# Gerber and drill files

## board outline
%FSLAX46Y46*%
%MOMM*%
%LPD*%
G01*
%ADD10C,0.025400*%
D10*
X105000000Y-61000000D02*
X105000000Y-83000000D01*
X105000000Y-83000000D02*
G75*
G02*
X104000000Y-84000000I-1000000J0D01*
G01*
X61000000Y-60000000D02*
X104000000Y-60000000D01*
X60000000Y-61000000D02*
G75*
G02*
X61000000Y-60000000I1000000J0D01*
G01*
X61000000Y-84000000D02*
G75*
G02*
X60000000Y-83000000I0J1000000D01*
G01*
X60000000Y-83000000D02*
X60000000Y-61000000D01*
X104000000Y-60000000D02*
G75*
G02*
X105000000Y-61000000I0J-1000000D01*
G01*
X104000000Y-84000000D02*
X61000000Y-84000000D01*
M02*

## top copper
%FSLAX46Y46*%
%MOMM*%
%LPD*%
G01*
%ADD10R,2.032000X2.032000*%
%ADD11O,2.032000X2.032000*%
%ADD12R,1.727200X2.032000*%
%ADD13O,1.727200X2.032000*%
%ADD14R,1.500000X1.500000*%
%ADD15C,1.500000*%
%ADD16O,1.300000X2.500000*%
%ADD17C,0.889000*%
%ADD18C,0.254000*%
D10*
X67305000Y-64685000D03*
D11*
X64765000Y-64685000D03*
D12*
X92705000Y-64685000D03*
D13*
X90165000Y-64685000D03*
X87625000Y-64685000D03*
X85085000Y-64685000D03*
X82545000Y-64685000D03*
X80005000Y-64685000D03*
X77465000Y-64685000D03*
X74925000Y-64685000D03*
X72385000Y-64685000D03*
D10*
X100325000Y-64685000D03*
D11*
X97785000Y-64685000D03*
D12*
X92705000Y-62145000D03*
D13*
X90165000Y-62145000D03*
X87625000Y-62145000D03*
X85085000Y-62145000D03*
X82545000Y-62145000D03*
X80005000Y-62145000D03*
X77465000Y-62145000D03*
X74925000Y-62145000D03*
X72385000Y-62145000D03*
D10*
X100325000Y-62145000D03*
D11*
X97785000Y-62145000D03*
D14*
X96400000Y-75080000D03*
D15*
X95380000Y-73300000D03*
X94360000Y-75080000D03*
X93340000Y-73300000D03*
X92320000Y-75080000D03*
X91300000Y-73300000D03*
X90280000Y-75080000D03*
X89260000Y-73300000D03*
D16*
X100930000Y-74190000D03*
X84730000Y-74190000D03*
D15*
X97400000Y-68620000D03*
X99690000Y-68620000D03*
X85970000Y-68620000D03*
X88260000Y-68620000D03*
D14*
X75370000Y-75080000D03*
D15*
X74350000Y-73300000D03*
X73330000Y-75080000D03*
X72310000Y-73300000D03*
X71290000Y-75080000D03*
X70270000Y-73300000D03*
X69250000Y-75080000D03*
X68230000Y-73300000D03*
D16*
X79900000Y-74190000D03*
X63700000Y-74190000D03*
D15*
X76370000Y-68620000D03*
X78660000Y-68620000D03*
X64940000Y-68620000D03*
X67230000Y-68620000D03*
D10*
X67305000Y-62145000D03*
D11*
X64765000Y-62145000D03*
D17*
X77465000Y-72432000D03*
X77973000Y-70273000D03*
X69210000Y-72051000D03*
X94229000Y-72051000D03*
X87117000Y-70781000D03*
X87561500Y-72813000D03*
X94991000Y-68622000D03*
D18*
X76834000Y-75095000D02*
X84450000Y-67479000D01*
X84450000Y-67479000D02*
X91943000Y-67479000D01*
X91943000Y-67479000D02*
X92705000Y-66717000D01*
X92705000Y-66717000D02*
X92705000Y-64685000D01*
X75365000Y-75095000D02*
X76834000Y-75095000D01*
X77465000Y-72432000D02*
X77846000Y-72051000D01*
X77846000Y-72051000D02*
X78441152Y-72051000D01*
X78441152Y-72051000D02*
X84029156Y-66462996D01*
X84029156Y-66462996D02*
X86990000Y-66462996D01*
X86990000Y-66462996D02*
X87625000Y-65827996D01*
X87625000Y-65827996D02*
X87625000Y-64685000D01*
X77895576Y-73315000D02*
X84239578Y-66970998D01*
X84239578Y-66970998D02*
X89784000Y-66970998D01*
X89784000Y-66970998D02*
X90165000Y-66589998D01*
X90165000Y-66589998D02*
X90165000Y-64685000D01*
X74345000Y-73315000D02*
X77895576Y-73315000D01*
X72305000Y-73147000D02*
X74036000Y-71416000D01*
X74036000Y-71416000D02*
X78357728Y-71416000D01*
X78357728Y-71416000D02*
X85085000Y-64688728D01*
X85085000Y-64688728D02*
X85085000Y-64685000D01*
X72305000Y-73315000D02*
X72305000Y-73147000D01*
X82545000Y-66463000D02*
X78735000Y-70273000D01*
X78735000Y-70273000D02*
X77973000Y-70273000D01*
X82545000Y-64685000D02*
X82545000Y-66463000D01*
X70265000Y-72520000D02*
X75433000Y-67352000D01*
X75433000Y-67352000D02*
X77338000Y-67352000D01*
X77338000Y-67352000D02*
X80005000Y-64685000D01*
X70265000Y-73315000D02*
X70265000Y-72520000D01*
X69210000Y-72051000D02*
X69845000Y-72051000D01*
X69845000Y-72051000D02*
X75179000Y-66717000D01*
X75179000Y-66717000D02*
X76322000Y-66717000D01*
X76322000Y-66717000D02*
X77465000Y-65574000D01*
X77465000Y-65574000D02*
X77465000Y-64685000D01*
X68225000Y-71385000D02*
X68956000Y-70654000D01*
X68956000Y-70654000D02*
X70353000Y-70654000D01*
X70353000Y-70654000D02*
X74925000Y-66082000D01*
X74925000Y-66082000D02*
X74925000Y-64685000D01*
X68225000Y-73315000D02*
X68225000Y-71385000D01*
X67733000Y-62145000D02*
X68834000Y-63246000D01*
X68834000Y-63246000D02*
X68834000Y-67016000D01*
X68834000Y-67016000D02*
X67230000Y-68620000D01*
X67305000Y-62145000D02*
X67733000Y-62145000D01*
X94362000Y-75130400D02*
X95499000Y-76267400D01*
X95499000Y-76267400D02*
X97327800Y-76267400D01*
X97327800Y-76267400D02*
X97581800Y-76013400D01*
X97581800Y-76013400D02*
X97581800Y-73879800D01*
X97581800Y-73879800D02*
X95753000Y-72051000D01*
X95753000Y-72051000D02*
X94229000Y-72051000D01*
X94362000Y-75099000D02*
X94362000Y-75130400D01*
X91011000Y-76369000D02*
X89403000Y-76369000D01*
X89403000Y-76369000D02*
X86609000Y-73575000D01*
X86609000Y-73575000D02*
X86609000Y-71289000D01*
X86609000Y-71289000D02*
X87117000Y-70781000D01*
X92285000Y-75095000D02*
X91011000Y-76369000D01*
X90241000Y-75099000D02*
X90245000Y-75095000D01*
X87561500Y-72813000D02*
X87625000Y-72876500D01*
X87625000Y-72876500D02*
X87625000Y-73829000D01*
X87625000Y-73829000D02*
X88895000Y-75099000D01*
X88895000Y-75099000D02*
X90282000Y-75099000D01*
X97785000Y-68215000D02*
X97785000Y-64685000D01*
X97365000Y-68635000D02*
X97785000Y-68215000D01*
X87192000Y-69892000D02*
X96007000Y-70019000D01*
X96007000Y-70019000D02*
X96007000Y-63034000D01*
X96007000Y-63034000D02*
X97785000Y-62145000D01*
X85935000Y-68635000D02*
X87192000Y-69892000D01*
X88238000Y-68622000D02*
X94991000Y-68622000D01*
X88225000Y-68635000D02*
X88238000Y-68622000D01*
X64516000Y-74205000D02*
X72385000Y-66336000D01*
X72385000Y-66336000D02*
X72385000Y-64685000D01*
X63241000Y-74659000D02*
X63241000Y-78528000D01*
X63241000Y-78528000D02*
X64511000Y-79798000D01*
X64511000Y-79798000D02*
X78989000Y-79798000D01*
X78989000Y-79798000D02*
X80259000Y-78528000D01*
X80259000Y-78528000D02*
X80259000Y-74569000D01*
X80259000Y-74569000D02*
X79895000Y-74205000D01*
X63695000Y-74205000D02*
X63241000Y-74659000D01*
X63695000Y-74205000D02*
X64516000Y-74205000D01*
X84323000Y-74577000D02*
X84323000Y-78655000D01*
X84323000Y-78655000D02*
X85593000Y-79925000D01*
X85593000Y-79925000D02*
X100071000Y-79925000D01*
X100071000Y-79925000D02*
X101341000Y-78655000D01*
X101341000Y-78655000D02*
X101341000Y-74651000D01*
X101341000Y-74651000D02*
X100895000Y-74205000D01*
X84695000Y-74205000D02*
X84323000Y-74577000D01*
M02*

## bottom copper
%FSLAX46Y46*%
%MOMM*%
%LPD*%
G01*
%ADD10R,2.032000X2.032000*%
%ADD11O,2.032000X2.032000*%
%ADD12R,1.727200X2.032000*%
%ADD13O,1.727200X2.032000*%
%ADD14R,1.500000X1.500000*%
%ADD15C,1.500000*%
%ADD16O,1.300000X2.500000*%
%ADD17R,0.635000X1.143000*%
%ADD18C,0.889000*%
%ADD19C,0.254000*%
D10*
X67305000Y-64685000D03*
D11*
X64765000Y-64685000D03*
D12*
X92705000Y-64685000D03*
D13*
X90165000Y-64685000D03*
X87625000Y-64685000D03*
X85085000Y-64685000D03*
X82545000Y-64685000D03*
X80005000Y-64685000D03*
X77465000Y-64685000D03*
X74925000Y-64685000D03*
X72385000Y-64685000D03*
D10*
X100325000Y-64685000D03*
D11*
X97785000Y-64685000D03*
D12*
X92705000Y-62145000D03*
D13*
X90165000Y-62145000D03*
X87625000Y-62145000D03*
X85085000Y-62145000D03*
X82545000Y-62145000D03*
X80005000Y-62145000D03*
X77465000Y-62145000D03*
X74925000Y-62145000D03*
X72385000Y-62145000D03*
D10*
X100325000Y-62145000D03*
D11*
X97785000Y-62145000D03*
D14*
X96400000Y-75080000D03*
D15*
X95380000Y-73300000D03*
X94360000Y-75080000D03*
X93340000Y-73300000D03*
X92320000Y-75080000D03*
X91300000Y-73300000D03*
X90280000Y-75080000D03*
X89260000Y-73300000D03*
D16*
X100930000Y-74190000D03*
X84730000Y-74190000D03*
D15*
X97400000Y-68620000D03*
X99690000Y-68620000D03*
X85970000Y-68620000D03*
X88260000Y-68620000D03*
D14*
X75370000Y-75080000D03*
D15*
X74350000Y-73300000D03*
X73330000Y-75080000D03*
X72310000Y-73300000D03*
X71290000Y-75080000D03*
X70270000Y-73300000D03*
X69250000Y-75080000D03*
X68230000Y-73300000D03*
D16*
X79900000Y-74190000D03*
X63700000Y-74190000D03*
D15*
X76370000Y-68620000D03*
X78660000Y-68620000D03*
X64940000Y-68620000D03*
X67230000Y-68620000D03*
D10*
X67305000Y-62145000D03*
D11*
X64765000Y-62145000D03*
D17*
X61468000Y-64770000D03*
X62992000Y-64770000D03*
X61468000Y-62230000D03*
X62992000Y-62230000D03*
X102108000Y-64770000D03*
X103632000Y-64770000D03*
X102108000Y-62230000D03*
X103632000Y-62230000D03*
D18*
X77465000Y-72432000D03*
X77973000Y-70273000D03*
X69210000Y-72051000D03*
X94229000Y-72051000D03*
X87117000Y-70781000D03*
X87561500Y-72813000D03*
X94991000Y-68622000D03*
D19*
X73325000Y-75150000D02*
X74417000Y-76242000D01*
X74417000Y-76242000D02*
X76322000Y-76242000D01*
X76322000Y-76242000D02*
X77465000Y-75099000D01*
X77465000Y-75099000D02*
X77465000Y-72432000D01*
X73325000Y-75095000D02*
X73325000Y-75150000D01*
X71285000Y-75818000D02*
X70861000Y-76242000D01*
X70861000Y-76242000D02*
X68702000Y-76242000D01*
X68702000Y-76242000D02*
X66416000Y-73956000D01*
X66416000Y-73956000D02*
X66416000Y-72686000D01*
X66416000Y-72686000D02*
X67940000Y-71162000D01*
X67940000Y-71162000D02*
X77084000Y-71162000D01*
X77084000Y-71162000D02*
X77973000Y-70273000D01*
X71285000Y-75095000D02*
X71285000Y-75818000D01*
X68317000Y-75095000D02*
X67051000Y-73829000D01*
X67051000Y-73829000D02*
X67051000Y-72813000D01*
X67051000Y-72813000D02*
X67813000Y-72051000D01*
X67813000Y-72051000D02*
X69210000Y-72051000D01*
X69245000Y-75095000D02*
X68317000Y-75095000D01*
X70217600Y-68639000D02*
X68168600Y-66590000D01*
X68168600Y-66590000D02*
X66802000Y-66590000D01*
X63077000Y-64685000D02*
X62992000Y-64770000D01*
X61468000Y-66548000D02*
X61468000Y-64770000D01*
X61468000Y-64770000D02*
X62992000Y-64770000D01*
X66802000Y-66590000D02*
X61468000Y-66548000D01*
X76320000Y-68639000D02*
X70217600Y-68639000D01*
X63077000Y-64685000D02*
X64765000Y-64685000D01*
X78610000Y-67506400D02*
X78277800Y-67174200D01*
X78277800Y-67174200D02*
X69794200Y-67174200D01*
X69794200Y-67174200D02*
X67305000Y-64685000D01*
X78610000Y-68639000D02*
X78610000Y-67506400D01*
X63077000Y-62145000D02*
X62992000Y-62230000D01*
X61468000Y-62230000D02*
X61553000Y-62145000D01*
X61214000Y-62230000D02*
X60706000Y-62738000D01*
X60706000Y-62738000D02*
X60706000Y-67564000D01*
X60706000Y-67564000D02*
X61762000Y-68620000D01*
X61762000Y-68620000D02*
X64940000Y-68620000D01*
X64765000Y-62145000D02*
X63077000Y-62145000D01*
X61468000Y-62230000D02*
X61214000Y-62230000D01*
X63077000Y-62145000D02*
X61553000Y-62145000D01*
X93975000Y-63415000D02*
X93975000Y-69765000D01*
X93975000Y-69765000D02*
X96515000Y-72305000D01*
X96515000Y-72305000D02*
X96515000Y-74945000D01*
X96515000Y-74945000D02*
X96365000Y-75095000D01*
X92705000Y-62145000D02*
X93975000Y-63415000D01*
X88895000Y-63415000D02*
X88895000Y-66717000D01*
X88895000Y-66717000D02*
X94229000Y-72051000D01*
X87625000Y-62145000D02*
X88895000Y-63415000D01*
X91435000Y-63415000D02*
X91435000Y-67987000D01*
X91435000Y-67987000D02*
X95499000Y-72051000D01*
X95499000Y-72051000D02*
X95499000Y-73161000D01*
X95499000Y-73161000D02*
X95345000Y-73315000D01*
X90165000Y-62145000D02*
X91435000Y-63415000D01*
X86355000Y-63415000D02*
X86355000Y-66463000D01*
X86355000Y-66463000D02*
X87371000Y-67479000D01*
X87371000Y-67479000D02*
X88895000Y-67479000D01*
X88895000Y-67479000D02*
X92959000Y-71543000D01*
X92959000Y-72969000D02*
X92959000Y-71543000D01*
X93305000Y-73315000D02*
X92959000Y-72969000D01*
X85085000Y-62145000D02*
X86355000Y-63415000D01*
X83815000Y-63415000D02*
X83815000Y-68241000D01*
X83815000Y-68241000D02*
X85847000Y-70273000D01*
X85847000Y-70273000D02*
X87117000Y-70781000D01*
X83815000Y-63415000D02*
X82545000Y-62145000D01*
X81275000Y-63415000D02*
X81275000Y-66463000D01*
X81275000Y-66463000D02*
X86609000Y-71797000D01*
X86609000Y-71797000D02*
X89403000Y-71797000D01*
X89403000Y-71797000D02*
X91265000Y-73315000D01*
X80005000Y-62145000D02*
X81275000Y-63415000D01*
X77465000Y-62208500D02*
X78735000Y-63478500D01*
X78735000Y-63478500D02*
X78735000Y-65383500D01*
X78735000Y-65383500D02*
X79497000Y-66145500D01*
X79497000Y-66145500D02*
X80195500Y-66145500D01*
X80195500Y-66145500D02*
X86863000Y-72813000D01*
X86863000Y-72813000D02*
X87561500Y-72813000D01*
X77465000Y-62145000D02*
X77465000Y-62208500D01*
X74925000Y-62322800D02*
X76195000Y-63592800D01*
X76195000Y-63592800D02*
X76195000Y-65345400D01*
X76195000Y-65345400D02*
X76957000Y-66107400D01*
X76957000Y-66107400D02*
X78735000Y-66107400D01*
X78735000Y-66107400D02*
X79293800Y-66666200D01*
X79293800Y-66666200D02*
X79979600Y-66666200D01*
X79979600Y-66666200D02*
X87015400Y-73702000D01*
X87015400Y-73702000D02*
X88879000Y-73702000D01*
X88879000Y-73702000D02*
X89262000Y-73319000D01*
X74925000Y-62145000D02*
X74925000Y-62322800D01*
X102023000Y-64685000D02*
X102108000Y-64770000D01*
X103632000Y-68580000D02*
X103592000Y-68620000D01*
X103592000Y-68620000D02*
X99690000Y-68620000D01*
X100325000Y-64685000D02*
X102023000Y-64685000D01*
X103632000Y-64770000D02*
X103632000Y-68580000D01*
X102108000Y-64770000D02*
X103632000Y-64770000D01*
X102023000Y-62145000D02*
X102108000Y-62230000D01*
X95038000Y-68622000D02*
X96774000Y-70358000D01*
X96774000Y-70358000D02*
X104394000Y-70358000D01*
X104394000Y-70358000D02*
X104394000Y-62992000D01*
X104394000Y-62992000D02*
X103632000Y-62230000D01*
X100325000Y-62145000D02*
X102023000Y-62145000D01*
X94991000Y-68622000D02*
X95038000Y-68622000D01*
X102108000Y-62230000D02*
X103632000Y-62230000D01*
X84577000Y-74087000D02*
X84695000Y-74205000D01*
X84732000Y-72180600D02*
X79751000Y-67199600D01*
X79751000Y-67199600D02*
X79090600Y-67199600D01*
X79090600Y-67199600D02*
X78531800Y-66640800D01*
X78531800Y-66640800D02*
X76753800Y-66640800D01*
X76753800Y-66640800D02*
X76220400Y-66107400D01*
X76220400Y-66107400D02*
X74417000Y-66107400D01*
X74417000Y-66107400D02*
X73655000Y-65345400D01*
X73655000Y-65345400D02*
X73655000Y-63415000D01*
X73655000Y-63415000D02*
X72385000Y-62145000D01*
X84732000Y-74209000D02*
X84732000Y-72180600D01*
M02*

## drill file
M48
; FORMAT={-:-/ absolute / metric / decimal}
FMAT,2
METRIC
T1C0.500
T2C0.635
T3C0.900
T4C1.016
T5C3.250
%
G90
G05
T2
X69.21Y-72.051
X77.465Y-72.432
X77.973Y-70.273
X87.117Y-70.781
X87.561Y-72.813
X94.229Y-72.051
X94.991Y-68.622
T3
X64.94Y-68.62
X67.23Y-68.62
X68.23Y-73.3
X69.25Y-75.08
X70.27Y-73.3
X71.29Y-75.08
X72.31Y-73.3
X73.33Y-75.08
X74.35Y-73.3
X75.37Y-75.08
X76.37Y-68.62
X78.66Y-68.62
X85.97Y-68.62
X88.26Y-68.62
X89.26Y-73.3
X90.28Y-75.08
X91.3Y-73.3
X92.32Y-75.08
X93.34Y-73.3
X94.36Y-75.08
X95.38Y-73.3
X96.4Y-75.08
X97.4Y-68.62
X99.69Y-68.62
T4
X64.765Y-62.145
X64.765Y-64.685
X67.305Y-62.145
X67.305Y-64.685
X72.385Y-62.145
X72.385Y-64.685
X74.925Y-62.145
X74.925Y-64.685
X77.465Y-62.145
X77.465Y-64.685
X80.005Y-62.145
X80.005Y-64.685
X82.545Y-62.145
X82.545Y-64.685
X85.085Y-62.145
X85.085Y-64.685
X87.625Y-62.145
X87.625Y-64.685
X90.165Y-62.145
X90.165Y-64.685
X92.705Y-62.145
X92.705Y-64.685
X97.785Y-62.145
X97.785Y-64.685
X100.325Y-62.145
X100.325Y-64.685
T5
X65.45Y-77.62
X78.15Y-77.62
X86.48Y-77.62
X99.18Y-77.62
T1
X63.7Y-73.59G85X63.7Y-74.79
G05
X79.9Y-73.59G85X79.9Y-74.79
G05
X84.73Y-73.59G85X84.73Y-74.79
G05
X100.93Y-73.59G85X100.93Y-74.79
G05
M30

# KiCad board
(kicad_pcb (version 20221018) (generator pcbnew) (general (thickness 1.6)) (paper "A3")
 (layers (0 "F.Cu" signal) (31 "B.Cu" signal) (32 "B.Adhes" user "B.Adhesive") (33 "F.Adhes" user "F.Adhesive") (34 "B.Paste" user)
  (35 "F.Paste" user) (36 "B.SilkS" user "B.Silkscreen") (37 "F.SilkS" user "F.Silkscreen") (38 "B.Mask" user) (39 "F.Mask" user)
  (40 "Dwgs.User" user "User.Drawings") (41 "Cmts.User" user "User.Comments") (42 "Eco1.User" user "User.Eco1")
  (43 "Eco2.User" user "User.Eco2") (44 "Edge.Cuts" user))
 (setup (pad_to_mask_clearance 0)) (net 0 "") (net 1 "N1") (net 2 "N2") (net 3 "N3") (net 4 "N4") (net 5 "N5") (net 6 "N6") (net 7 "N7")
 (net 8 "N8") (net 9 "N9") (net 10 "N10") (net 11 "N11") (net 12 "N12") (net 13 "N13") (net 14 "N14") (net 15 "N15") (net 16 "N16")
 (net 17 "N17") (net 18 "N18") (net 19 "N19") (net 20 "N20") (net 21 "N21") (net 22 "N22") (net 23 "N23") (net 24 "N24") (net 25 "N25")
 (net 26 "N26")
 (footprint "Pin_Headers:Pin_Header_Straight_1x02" (layer "F.Cu") (at 66.035 64.685 180)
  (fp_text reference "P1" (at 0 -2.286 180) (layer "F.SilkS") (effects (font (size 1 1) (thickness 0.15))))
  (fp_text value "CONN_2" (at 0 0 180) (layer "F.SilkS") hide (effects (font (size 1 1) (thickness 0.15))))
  (pad "1" thru_hole rect (at -1.27 0 180) (size 2.032 2.032) (drill 1.016) (layers "*.Cu" "*.Mask" "F.SilkS") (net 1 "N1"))
  (pad "2" thru_hole oval (at 1.27 0 180) (size 2.032 2.032) (drill 1.016) (layers "*.Cu" "*.Mask" "F.SilkS") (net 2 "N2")))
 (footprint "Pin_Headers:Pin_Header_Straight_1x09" (layer "F.Cu") (at 82.545 64.685 180)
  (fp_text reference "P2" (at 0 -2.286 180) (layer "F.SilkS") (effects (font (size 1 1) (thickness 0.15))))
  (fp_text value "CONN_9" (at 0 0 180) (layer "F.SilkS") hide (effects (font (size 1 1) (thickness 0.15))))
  (pad "1" thru_hole rect (at -10.16 0 180) (size 1.7272 2.032) (drill 1.016) (layers "*.Cu" "*.Mask" "F.SilkS") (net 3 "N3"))
  (pad "2" thru_hole oval (at -7.62 0 180) (size 1.7272 2.032) (drill 1.016) (layers "*.Cu" "*.Mask" "F.SilkS") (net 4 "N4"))
  (pad "3" thru_hole oval (at -5.08 0 180) (size 1.7272 2.032) (drill 1.016) (layers "*.Cu" "*.Mask" "F.SilkS") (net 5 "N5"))
  (pad "4" thru_hole oval (at -2.54 0 180) (size 1.7272 2.032) (drill 1.016) (layers "*.Cu" "*.Mask" "F.SilkS") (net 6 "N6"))
  (pad "5" thru_hole oval (at 0 0 180) (size 1.7272 2.032) (drill 1.016) (layers "*.Cu" "*.Mask" "F.SilkS") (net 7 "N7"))
  (pad "6" thru_hole oval (at 2.54 0 180) (size 1.7272 2.032) (drill 1.016) (layers "*.Cu" "*.Mask" "F.SilkS") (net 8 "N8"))
  (pad "7" thru_hole oval (at 5.08 0 180) (size 1.7272 2.032) (drill 1.016) (layers "*.Cu" "*.Mask" "F.SilkS") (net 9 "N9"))
  (pad "8" thru_hole oval (at 7.62 0 180) (size 1.7272 2.032) (drill 1.016) (layers "*.Cu" "*.Mask" "F.SilkS") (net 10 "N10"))
  (pad "9" thru_hole oval (at 10.16 0 180) (size 1.7272 2.032) (drill 1.016) (layers "*.Cu" "*.Mask" "F.SilkS") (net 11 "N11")))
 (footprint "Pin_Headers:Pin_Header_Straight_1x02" (layer "F.Cu") (at 99.055 64.685 180)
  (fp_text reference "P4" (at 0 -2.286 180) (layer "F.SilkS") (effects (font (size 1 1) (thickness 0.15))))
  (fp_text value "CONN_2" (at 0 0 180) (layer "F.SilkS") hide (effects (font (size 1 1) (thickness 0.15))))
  (pad "1" thru_hole rect (at -1.27 0 180) (size 2.032 2.032) (drill 1.016) (layers "*.Cu" "*.Mask" "F.SilkS") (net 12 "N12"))
  (pad "2" thru_hole oval (at 1.27 0 180) (size 2.032 2.032) (drill 1.016) (layers "*.Cu" "*.Mask" "F.SilkS") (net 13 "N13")))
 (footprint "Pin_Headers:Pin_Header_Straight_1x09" (layer "F.Cu") (at 82.545 62.145 180)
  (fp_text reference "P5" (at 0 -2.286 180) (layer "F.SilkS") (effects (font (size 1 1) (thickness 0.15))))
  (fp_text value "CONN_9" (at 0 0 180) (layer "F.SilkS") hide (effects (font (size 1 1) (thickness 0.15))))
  (pad "1" thru_hole rect (at -10.16 0 180) (size 1.7272 2.032) (drill 1.016) (layers "*.Cu" "*.Mask" "F.SilkS") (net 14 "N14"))
  (pad "2" thru_hole oval (at -7.62 0 180) (size 1.7272 2.032) (drill 1.016) (layers "*.Cu" "*.Mask" "F.SilkS") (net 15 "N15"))
  (pad "3" thru_hole oval (at -5.08 0 180) (size 1.7272 2.032) (drill 1.016) (layers "*.Cu" "*.Mask" "F.SilkS") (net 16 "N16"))
  (pad "4" thru_hole oval (at -2.54 0 180) (size 1.7272 2.032) (drill 1.016) (layers "*.Cu" "*.Mask" "F.SilkS") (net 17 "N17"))
  (pad "5" thru_hole oval (at 0 0 180) (size 1.7272 2.032) (drill 1.016) (layers "*.Cu" "*.Mask" "F.SilkS") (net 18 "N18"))
  (pad "6" thru_hole oval (at 2.54 0 180) (size 1.7272 2.032) (drill 1.016) (layers "*.Cu" "*.Mask" "F.SilkS") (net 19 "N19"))
  (pad "7" thru_hole oval (at 5.08 0 180) (size 1.7272 2.032) (drill 1.016) (layers "*.Cu" "*.Mask" "F.SilkS") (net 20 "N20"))
  (pad "8" thru_hole oval (at 7.62 0 180) (size 1.7272 2.032) (drill 1.016) (layers "*.Cu" "*.Mask" "F.SilkS") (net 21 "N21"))
  (pad "9" thru_hole oval (at 10.16 0 180) (size 1.7272 2.032) (drill 1.016) (layers "*.Cu" "*.Mask" "F.SilkS") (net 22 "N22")))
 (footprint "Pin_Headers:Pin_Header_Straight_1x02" (layer "F.Cu") (at 99.055 62.145 180)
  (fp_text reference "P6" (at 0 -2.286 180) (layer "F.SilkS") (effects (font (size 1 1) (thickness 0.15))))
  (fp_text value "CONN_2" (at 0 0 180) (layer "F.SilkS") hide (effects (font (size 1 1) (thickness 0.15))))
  (pad "1" thru_hole rect (at -1.27 0 180) (size 2.032 2.032) (drill 1.016) (layers "*.Cu" "*.Mask" "F.SilkS") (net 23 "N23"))
  (pad "2" thru_hole oval (at 1.27 0 180) (size 2.032 2.032) (drill 1.016) (layers "*.Cu" "*.Mask" "F.SilkS") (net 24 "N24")))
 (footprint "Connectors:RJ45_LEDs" (layer "F.Cu") (at 96.4 75.08 180)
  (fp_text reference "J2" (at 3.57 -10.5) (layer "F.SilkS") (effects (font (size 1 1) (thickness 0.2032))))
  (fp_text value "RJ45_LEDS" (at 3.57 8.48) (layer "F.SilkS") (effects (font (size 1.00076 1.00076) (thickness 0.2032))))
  (pad "" np_thru_hole circle (at -2.78 -2.54) (size 3.25 3.25) (drill 3.25) (layers "*.Cu" "*.Mask" "F.SilkS"))
  (pad "" np_thru_hole circle (at 9.92 -2.54) (size 3.25 3.25) (drill 3.25) (layers "*.Cu" "*.Mask" "F.SilkS"))
  (pad "1" thru_hole rect (at 0 0) (size 1.5 1.5) (drill 0.9) (layers "*.Cu" "*.Mask" "F.SilkS") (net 14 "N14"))
  (pad "2" thru_hole circle (at 1.02 1.78) (size 1.5 1.5) (drill 0.9) (layers "*.Cu" "*.Mask" "F.SilkS") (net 15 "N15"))
  (pad "3" thru_hole circle (at 2.04 0) (size 1.5 1.5) (drill 0.9) (layers "*.Cu" "*.Mask" "F.SilkS") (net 16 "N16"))
  (pad "4" thru_hole circle (at 3.06 1.78) (size 1.5 1.5) (drill 0.9) (layers "*.Cu" "*.Mask" "F.SilkS") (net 17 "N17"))
  (pad "5" thru_hole circle (at 4.08 0) (size 1.5 1.5) (drill 0.9) (layers "*.Cu" "*.Mask" "F.SilkS") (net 18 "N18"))
  (pad "6" thru_hole circle (at 5.1 1.78) (size 1.5 1.5) (drill 0.9) (layers "*.Cu" "*.Mask" "F.SilkS") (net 19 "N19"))
  (pad "7" thru_hole circle (at 6.12 0) (size 1.5 1.5) (drill 0.9) (layers "*.Cu" "*.Mask" "F.SilkS") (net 20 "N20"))
  (pad "8" thru_hole circle (at 7.14 1.78) (size 1.5 1.5) (drill 0.9) (layers "*.Cu" "*.Mask" "F.SilkS") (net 21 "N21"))
  (pad "13" thru_hole oval (at -4.53 0.89) (size 1.3 2.5) (drill oval 0.5 1.7) (layers "*.Cu" "*.Mask" "F.SilkS") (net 22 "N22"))
  (pad "13" thru_hole oval (at 11.67 0.89) (size 1.3 2.5) (drill oval 0.5 1.7) (layers "*.Cu" "*.Mask" "F.SilkS") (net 22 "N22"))
  (pad "GA" thru_hole circle (at -1 6.46) (size 1.5 1.5) (drill 0.9) (layers "*.Cu" "*.Mask" "F.SilkS") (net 13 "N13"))
  (pad "GK" thru_hole circle (at -3.29 6.46) (size 1.5 1.5) (drill 0.9) (layers "*.Cu" "*.Mask" "F.SilkS") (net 12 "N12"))
  (pad "YA" thru_hole circle (at 10.43 6.46) (size 1.5 1.5) (drill 0.9) (layers "*.Cu" "*.Mask" "F.SilkS") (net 24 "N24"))
  (pad "YK" thru_hole circle (at 8.14 6.46) (size 1.5 1.5) (drill 0.9) (layers "*.Cu" "*.Mask" "F.SilkS") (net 23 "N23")))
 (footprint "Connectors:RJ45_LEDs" (layer "F.Cu") (at 75.37 75.08 180)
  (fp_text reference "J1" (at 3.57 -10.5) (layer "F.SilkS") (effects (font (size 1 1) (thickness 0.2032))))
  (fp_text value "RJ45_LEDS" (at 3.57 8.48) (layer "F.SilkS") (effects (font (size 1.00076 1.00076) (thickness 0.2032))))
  (pad "" np_thru_hole circle (at -2.78 -2.54) (size 3.25 3.25) (drill 3.25) (layers "*.Cu" "*.Mask" "F.SilkS"))
  (pad "" np_thru_hole circle (at 9.92 -2.54) (size 3.25 3.25) (drill 3.25) (layers "*.Cu" "*.Mask" "F.SilkS"))
  (pad "1" thru_hole rect (at 0 0) (size 1.5 1.5) (drill 0.9) (layers "*.Cu" "*.Mask" "F.SilkS") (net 3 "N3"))
  (pad "2" thru_hole circle (at 1.02 1.78) (size 1.5 1.5) (drill 0.9) (layers "*.Cu" "*.Mask" "F.SilkS") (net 4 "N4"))
  (pad "3" thru_hole circle (at 2.04 0) (size 1.5 1.5) (drill 0.9) (layers "*.Cu" "*.Mask" "F.SilkS") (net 5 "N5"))
  (pad "4" thru_hole circle (at 3.06 1.78) (size 1.5 1.5) (drill 0.9) (layers "*.Cu" "*.Mask" "F.SilkS") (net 6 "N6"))
  (pad "5" thru_hole circle (at 4.08 0) (size 1.5 1.5) (drill 0.9) (layers "*.Cu" "*.Mask" "F.SilkS") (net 7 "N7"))
  (pad "6" thru_hole circle (at 5.1 1.78) (size 1.5 1.5) (drill 0.9) (layers "*.Cu" "*.Mask" "F.SilkS") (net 8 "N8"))
  (pad "7" thru_hole circle (at 6.12 0) (size 1.5 1.5) (drill 0.9) (layers "*.Cu" "*.Mask" "F.SilkS") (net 9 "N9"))
  (pad "8" thru_hole circle (at 7.14 1.78) (size 1.5 1.5) (drill 0.9) (layers "*.Cu" "*.Mask" "F.SilkS") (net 10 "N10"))
  (pad "13" thru_hole oval (at -4.53 0.89) (size 1.3 2.5) (drill oval 0.5 1.7) (layers "*.Cu" "*.Mask" "F.SilkS") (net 11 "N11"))
  (pad "13" thru_hole oval (at 11.67 0.89) (size 1.3 2.5) (drill oval 0.5 1.7) (layers "*.Cu" "*.Mask" "F.SilkS") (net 11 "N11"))
  (pad "GA" thru_hole circle (at -1 6.46) (size 1.5 1.5) (drill 0.9) (layers "*.Cu" "*.Mask" "F.SilkS") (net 2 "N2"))
  (pad "GK" thru_hole circle (at -3.29 6.46) (size 1.5 1.5) (drill 0.9) (layers "*.Cu" "*.Mask" "F.SilkS") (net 1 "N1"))
  (pad "YA" thru_hole circle (at 10.43 6.46) (size 1.5 1.5) (drill 0.9) (layers "*.Cu" "*.Mask" "F.SilkS") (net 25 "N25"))
  (pad "YK" thru_hole circle (at 8.14 6.46) (size 1.5 1.5) (drill 0.9) (layers "*.Cu" "*.Mask" "F.SilkS") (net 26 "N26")))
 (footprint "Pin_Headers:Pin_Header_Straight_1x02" (layer "F.Cu") (at 66.035 62.145 180)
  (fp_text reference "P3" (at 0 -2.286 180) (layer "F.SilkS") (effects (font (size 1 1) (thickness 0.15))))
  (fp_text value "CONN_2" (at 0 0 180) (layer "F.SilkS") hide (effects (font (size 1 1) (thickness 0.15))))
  (pad "1" thru_hole rect (at -1.27 0 180) (size 2.032 2.032) (drill 1.016) (layers "*.Cu" "*.Mask" "F.SilkS") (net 26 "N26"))
  (pad "2" thru_hole oval (at 1.27 0 180) (size 2.032 2.032) (drill 1.016) (layers "*.Cu" "*.Mask" "F.SilkS") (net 25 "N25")))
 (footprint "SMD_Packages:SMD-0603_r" (layer "B.Cu") (at 62.23 64.77)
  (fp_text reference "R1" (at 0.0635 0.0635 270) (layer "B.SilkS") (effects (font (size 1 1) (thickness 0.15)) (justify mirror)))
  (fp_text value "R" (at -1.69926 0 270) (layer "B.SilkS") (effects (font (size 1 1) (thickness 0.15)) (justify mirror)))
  (pad "1" smd rect (at -0.762 0) (size 0.635 1.143) (layers "B.Cu" "B.Paste" "B.Mask") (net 2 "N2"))
  (pad "2" smd rect (at 0.762 0) (size 0.635 1.143) (layers "B.Cu" "B.Paste" "B.Mask") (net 2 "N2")))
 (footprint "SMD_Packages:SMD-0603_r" (layer "B.Cu") (at 62.23 62.23)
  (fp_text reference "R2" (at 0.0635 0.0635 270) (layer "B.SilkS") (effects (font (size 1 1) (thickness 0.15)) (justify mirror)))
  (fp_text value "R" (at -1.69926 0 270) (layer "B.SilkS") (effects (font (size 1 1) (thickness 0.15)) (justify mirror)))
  (pad "1" smd rect (at -0.762 0) (size 0.635 1.143) (layers "B.Cu" "B.Paste" "B.Mask") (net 25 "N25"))
  (pad "2" smd rect (at 0.762 0) (size 0.635 1.143) (layers "B.Cu" "B.Paste" "B.Mask") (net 25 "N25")))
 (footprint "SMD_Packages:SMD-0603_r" (layer "B.Cu") (at 102.87 64.77)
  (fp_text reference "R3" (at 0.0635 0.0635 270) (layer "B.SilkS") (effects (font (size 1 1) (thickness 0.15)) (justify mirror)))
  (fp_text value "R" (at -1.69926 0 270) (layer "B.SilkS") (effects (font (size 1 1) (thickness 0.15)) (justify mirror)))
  (pad "1" smd rect (at -0.762 0) (size 0.635 1.143) (layers "B.Cu" "B.Paste" "B.Mask") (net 12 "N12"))
  (pad "2" smd rect (at 0.762 0) (size 0.635 1.143) (layers "B.Cu" "B.Paste" "B.Mask") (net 12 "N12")))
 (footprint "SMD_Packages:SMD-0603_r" (layer "B.Cu") (at 102.87 62.23)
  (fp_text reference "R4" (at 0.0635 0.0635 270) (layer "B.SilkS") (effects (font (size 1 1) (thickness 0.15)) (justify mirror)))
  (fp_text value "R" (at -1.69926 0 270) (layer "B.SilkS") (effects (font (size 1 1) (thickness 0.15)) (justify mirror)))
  (pad "1" smd rect (at -0.762 0) (size 0.635 1.143) (layers "B.Cu" "B.Paste" "B.Mask") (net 23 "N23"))
  (pad "2" smd rect (at 0.762 0) (size 0.635 1.143) (layers "B.Cu" "B.Paste" "B.Mask") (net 23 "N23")))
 (gr_line (start 105 61) (end 105 83) (stroke (width 0.0254) (type solid)) (layer "Edge.Cuts"))
 (gr_arc (start 105 83) (mid 104.707107 83.707107) (end 104 84) (stroke (width 0.0254) (type solid)) (layer "Edge.Cuts"))
 (gr_line (start 61 60) (end 104 60) (stroke (width 0.0254) (type solid)) (layer "Edge.Cuts"))
 (gr_arc (start 60 61) (mid 60.292893 60.292893) (end 61 60) (stroke (width 0.0254) (type solid)) (layer "Edge.Cuts"))
 (gr_arc (start 61 84) (mid 60.292893 83.707107) (end 60 83) (stroke (width 0.0254) (type solid)) (layer "Edge.Cuts"))
 (gr_line (start 60 83) (end 60 61) (stroke (width 0.0254) (type solid)) (layer "Edge.Cuts"))
 (gr_arc (start 104 60) (mid 104.707107 60.292893) (end 105 61) (stroke (width 0.0254) (type solid)) (layer "Edge.Cuts"))
 (gr_line (start 104 84) (end 61 84) (stroke (width 0.0254) (type solid)) (layer "Edge.Cuts"))
 (segment (start 76.834 75.095) (end 84.45 67.479) (width 0.254) (layer "F.Cu") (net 3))
 (segment (start 84.45 67.479) (end 91.943 67.479) (width 0.254) (layer "F.Cu") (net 3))
 (segment (start 91.943 67.479) (end 92.705 66.717) (width 0.254) (layer "F.Cu") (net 3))
 (segment (start 92.705 66.717) (end 92.705 64.685) (width 0.254) (layer "F.Cu") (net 3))
 (segment (start 75.365 75.095) (end 76.834 75.095) (width 0.254) (layer "F.Cu") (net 3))
 (segment (start 77.465 72.432) (end 77.846 72.051) (width 0.254) (layer "F.Cu") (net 5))
 (segment (start 77.846 72.051) (end 78.441152 72.051) (width 0.254) (layer "F.Cu") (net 5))
 (segment (start 78.441152 72.051) (end 84.029156 66.462996) (width 0.254) (layer "F.Cu") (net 5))
 (segment (start 84.029156 66.462996) (end 86.99 66.462996) (width 0.254) (layer "F.Cu") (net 5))
 (segment (start 86.99 66.462996) (end 87.625 65.827996) (width 0.254) (layer "F.Cu") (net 5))
 (segment (start 87.625 65.827996) (end 87.625 64.685) (width 0.254) (layer "F.Cu") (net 5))
 (via (at 77.465 72.432) (size 0.889) (drill 0.635) (layers "F.Cu" "B.Cu") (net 5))
 (segment (start 73.325 75.15) (end 74.417 76.242) (width 0.254) (layer "B.Cu") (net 5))
 (segment (start 74.417 76.242) (end 76.322 76.242) (width 0.254) (layer "B.Cu") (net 5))
 (segment (start 76.322 76.242) (end 77.465 75.099) (width 0.254) (layer "B.Cu") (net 5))
 (segment (start 77.465 75.099) (end 77.465 72.432) (width 0.254) (layer "B.Cu") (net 5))
 (segment (start 73.325 75.095) (end 73.325 75.15) (width 0.254) (layer "B.Cu") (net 5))
 (segment (start 77.895576 73.315) (end 84.239578 66.970998) (width 0.254) (layer "F.Cu") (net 4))
 (segment (start 84.239578 66.970998) (end 89.784 66.970998) (width 0.254) (layer "F.Cu") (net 4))
 (segment (start 89.784 66.970998) (end 90.165 66.589998) (width 0.254) (layer "F.Cu") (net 4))
 (segment (start 90.165 66.589998) (end 90.165 64.685) (width 0.254) (layer "F.Cu") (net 4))
 (segment (start 74.345 73.315) (end 77.895576 73.315) (width 0.254) (layer "F.Cu") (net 4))
 (segment (start 72.305 73.147) (end 74.036 71.416) (width 0.254) (layer "F.Cu") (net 6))
 (segment (start 74.036 71.416) (end 78.357728 71.416) (width 0.254) (layer "F.Cu") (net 6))
 (segment (start 78.357728 71.416) (end 85.085 64.688728) (width 0.254) (layer "F.Cu") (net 6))
 (segment (start 85.085 64.688728) (end 85.085 64.685) (width 0.254) (layer "F.Cu") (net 6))
 (segment (start 72.305 73.315) (end 72.305 73.147) (width 0.254) (layer "F.Cu") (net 6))
 (segment (start 82.545 66.463) (end 78.735 70.273) (width 0.254) (layer "F.Cu") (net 7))
 (segment (start 78.735 70.273) (end 77.973 70.273) (width 0.254) (layer "F.Cu") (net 7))
 (segment (start 82.545 64.685) (end 82.545 66.463) (width 0.254) (layer "F.Cu") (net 7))
 (via (at 77.973 70.273) (size 0.889) (drill 0.635) (layers "F.Cu" "B.Cu") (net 7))
 (segment (start 71.285 75.818) (end 70.861 76.242) (width 0.254) (layer "B.Cu") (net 7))
 (segment (start 70.861 76.242) (end 68.702 76.242) (width 0.254) (layer "B.Cu") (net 7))
 (segment (start 68.702 76.242) (end 66.416 73.956) (width 0.254) (layer "B.Cu") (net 7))
 (segment (start 66.416 73.956) (end 66.416 72.686) (width 0.254) (layer "B.Cu") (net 7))
 (segment (start 66.416 72.686) (end 67.94 71.162) (width 0.254) (layer "B.Cu") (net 7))
 (segment (start 67.94 71.162) (end 77.084 71.162) (width 0.254) (layer "B.Cu") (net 7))
 (segment (start 77.084 71.162) (end 77.973 70.273) (width 0.254) (layer "B.Cu") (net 7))
 (segment (start 71.285 75.095) (end 71.285 75.818) (width 0.254) (layer "B.Cu") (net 7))
 (segment (start 70.265 72.52) (end 75.433 67.352) (width 0.254) (layer "F.Cu") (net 8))
 (segment (start 75.433 67.352) (end 77.338 67.352) (width 0.254) (layer "F.Cu") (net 8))
 (segment (start 77.338 67.352) (end 80.005 64.685) (width 0.254) (layer "F.Cu") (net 8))
 (segment (start 70.265 73.315) (end 70.265 72.52) (width 0.254) (layer "F.Cu") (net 8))
 (segment (start 69.21 72.051) (end 69.845 72.051) (width 0.254) (layer "F.Cu") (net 9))
 (segment (start 69.845 72.051) (end 75.179 66.717) (width 0.254) (layer "F.Cu") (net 9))
 (segment (start 75.179 66.717) (end 76.322 66.717) (width 0.254) (layer "F.Cu") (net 9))
 (segment (start 76.322 66.717) (end 77.465 65.574) (width 0.254) (layer "F.Cu") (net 9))
 (segment (start 77.465 65.574) (end 77.465 64.685) (width 0.254) (layer "F.Cu") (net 9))
 (via (at 69.21 72.051) (size 0.889) (drill 0.635) (layers "F.Cu" "B.Cu") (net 9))
 (segment (start 68.317 75.095) (end 67.051 73.829) (width 0.254) (layer "B.Cu") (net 9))
 (segment (start 67.051 73.829) (end 67.051 72.813) (width 0.254) (layer "B.Cu") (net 9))
 (segment (start 67.051 72.813) (end 67.813 72.051) (width 0.254) (layer "B.Cu") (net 9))
 (segment (start 67.813 72.051) (end 69.21 72.051) (width 0.254) (layer "B.Cu") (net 9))
 (segment (start 69.245 75.095) (end 68.317 75.095) (width 0.254) (layer "B.Cu") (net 9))
 (segment (start 68.225 71.385) (end 68.956 70.654) (width 0.254) (layer "F.Cu") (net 10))
 (segment (start 68.956 70.654) (end 70.353 70.654) (width 0.254) (layer "F.Cu") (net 10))
 (segment (start 70.353 70.654) (end 74.925 66.082) (width 0.254) (layer "F.Cu") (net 10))
 (segment (start 74.925 66.082) (end 74.925 64.685) (width 0.254) (layer "F.Cu") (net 10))
 (segment (start 68.225 73.315) (end 68.225 71.385) (width 0.254) (layer "F.Cu") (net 10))
 (segment (start 70.2176 68.639) (end 68.1686 66.59) (width 0.254) (layer "B.Cu") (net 2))
 (segment (start 68.1686 66.59) (end 66.802 66.59) (width 0.254) (layer "B.Cu") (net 2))
 (segment (start 63.077 64.685) (end 62.992 64.77) (width 0.254) (layer "B.Cu") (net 2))
 (segment (start 61.468 66.548) (end 61.468 64.77) (width 0.254) (layer "B.Cu") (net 2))
 (segment (start 61.468 64.77) (end 62.992 64.77) (width 0.254) (layer "B.Cu") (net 2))
 (segment (start 66.802 66.59) (end 61.468 66.548) (width 0.254) (layer "B.Cu") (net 2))
 (segment (start 76.32 68.639) (end 70.2176 68.639) (width 0.254) (layer "B.Cu") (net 2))
 (segment (start 63.077 64.685) (end 64.765 64.685) (width 0.254) (layer "B.Cu") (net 2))
 (segment (start 78.61 67.5064) (end 78.2778 67.1742) (width 0.254) (layer "B.Cu") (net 1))
 (segment (start 78.2778 67.1742) (end 69.7942 67.1742) (width 0.254) (layer "B.Cu") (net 1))
 (segment (start 69.7942 67.1742) (end 67.305 64.685) (width 0.254) (layer "B.Cu") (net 1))
 (segment (start 78.61 68.639) (end 78.61 67.5064) (width 0.254) (layer "B.Cu") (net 1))
 (segment (start 63.077 62.145) (end 62.992 62.23) (width 0.254) (layer "B.Cu") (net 25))
 (segment (start 61.468 62.23) (end 61.553 62.145) (width 0.254) (layer "B.Cu") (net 25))
 (segment (start 61.214 62.23) (end 60.706 62.738) (width 0.254) (layer "B.Cu") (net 25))
 (segment (start 60.706 62.738) (end 60.706 67.564) (width 0.254) (layer "B.Cu") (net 25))
 (segment (start 60.706 67.564) (end 61.762 68.62) (width 0.254) (layer "B.Cu") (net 25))
 (segment (start 61.762 68.62) (end 64.94 68.62) (width 0.254) (layer "B.Cu") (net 25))
 (segment (start 64.765 62.145) (end 63.077 62.145) (width 0.254) (layer "B.Cu") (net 25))
 (segment (start 61.468 62.23) (end 61.214 62.23) (width 0.254) (layer "B.Cu") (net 25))
 (segment (start 63.077 62.145) (end 61.553 62.145) (width 0.254) (layer "B.Cu") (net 25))
 (segment (start 67.733 62.145) (end 68.834 63.246) (width 0.254) (layer "F.Cu") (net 26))
 (segment (start 68.834 63.246) (end 68.834 67.016) (width 0.254) (layer "F.Cu") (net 26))
 (segment (start 68.834 67.016) (end 67.23 68.62) (width 0.254) (layer "F.Cu") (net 26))
 (segment (start 67.305 62.145) (end 67.733 62.145) (width 0.254) (layer "F.Cu") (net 26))
 (segment (start 93.975 63.415) (end 93.975 69.765) (width 0.254) (layer "B.Cu") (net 14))
 (segment (start 93.975 69.765) (end 96.515 72.305) (width 0.254) (layer "B.Cu") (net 14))
 (segment (start 96.515 72.305) (end 96.515 74.945) (width 0.254) (layer "B.Cu") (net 14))
 (segment (start 96.515 74.945) (end 96.365 75.095) (width 0.254) (layer "B.Cu") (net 14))
 (segment (start 92.705 62.145) (end 93.975 63.415) (width 0.254) (layer "B.Cu") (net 14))
 (segment (start 94.362 75.1304) (end 95.499 76.2674) (width 0.254) (layer "F.Cu") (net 16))
 (segment (start 95.499 76.2674) (end 97.3278 76.2674) (width 0.254) (layer "F.Cu") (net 16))
 (segment (start 97.3278 76.2674) (end 97.5818 76.0134) (width 0.254) (layer "F.Cu") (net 16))
 (segment (start 97.5818 76.0134) (end 97.5818 73.8798) (width 0.254) (layer "F.Cu") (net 16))
 (segment (start 97.5818 73.8798) (end 95.753 72.051) (width 0.254) (layer "F.Cu") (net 16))
 (segment (start 95.753 72.051) (end 94.229 72.051) (width 0.254) (layer "F.Cu") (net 16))
 (segment (start 94.362 75.099) (end 94.362 75.1304) (width 0.254) (layer "F.Cu") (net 16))
 (via (at 94.229 72.051) (size 0.889) (drill 0.635) (layers "F.Cu" "B.Cu") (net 16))
 (segment (start 88.895 63.415) (end 88.895 66.717) (width 0.254) (layer "B.Cu") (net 16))
 (segment (start 88.895 66.717) (end 94.229 72.051) (width 0.254) (layer "B.Cu") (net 16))
 (segment (start 87.625 62.145) (end 88.895 63.415) (width 0.254) (layer "B.Cu") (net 16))
 (segment (start 91.435 63.415) (end 91.435 67.987) (width 0.254) (layer "B.Cu") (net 15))
 (segment (start 91.435 67.987) (end 95.499 72.051) (width 0.254) (layer "B.Cu") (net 15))
 (segment (start 95.499 72.051) (end 95.499 73.161) (width 0.254) (layer "B.Cu") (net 15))
 (segment (start 95.499 73.161) (end 95.345 73.315) (width 0.254) (layer "B.Cu") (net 15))
 (segment (start 90.165 62.145) (end 91.435 63.415) (width 0.254) (layer "B.Cu") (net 15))
 (segment (start 86.355 63.415) (end 86.355 66.463) (width 0.254) (layer "B.Cu") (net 17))
 (segment (start 86.355 66.463) (end 87.371 67.479) (width 0.254) (layer "B.Cu") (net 17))
 (segment (start 87.371 67.479) (end 88.895 67.479) (width 0.254) (layer "B.Cu") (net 17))
 (segment (start 88.895 67.479) (end 92.959 71.543) (width 0.254) (layer "B.Cu") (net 17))
 (segment (start 92.959 72.969) (end 92.959 71.543) (width 0.254) (layer "B.Cu") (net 17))
 (segment (start 93.305 73.315) (end 92.959 72.969) (width 0.254) (layer "B.Cu") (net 17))
 (segment (start 85.085 62.145) (end 86.355 63.415) (width 0.254) (layer "B.Cu") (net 17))
 (segment (start 91.011 76.369) (end 89.403 76.369) (width 0.254) (layer "F.Cu") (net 18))
 (segment (start 89.403 76.369) (end 86.609 73.575) (width 0.254) (layer "F.Cu") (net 18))
 (segment (start 86.609 73.575) (end 86.609 71.289) (width 0.254) (layer "F.Cu") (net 18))
 (segment (start 86.609 71.289) (end 87.117 70.781) (width 0.254) (layer "F.Cu") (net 18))
 (segment (start 92.285 75.095) (end 91.011 76.369) (width 0.254) (layer "F.Cu") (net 18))
 (via (at 87.117 70.781) (size 0.889) (drill 0.635) (layers "F.Cu" "B.Cu") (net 18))
 (segment (start 83.815 63.415) (end 83.815 68.241) (width 0.254) (layer "B.Cu") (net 18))
 (segment (start 83.815 68.241) (end 85.847 70.273) (width 0.254) (layer "B.Cu") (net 18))
 (segment (start 85.847 70.273) (end 87.117 70.781) (width 0.254) (layer "B.Cu") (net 18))
 (segment (start 83.815 63.415) (end 82.545 62.145) (width 0.254) (layer "B.Cu") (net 18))
 (segment (start 81.275 63.415) (end 81.275 66.463) (width 0.254) (layer "B.Cu") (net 19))
 (segment (start 81.275 66.463) (end 86.609 71.797) (width 0.254) (layer "B.Cu") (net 19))
 (segment (start 86.609 71.797) (end 89.403 71.797) (width 0.254) (layer "B.Cu") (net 19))
 (segment (start 89.403 71.797) (end 91.265 73.315) (width 0.254) (layer "B.Cu") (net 19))
 (segment (start 80.005 62.145) (end 81.275 63.415) (width 0.254) (layer "B.Cu") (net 19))
 (segment (start 90.241 75.099) (end 90.245 75.095) (width 0.254) (layer "F.Cu") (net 20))
 (segment (start 87.5615 72.813) (end 87.625 72.8765) (width 0.254) (layer "F.Cu") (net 20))
 (segment (start 87.625 72.8765) (end 87.625 73.829) (width 0.254) (layer "F.Cu") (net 20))
 (segment (start 87.625 73.829) (end 88.895 75.099) (width 0.254) (layer "F.Cu") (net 20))
 (segment (start 88.895 75.099) (end 90.282 75.099) (width 0.254) (layer "F.Cu") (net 20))
 (via (at 87.5615 72.813) (size 0.889) (drill 0.635) (layers "F.Cu" "B.Cu") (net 20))
 (segment (start 77.465 62.2085) (end 78.735 63.4785) (width 0.254) (layer "B.Cu") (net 20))
 (segment (start 78.735 63.4785) (end 78.735 65.3835) (width 0.254) (layer "B.Cu") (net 20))
 (segment (start 78.735 65.3835) (end 79.497 66.1455) (width 0.254) (layer "B.Cu") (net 20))
 (segment (start 79.497 66.1455) (end 80.1955 66.1455) (width 0.254) (layer "B.Cu") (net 20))
 (segment (start 80.1955 66.1455) (end 86.863 72.813) (width 0.254) (layer "B.Cu") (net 20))
 (segment (start 86.863 72.813) (end 87.5615 72.813) (width 0.254) (layer "B.Cu") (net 20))
 (segment (start 77.465 62.145) (end 77.465 62.2085) (width 0.254) (layer "B.Cu") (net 20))
 (segment (start 74.925 62.3228) (end 76.195 63.5928) (width 0.254) (layer "B.Cu") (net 21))
 (segment (start 76.195 63.5928) (end 76.195 65.3454) (width 0.254) (layer "B.Cu") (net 21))
 (segment (start 76.195 65.3454) (end 76.957 66.1074) (width 0.254) (layer "B.Cu") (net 21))
 (segment (start 76.957 66.1074) (end 78.735 66.1074) (width 0.254) (layer "B.Cu") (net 21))
 (segment (start 78.735 66.1074) (end 79.2938 66.6662) (width 0.254) (layer "B.Cu") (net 21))
 (segment (start 79.2938 66.6662) (end 79.9796 66.6662) (width 0.254) (layer "B.Cu") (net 21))
 (segment (start 79.9796 66.6662) (end 87.0154 73.702) (width 0.254) (layer "B.Cu") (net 21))
 (segment (start 87.0154 73.702) (end 88.879 73.702) (width 0.254) (layer "B.Cu") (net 21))
 (segment (start 88.879 73.702) (end 89.262 73.319) (width 0.254) (layer "B.Cu") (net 21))
 (segment (start 74.925 62.145) (end 74.925 62.3228) (width 0.254) (layer "B.Cu") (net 21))
 (segment (start 97.785 68.215) (end 97.785 64.685) (width 0.254) (layer "F.Cu") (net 13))
 (segment (start 97.365 68.635) (end 97.785 68.215) (width 0.254) (layer "F.Cu") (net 13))
 (segment (start 102.023 64.685) (end 102.108 64.77) (width 0.254) (layer "B.Cu") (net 12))
 (segment (start 103.632 68.58) (end 103.592 68.62) (width 0.254) (layer "B.Cu") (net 12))
 (segment (start 103.592 68.62) (end 99.69 68.62) (width 0.254) (layer "B.Cu") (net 12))
 (segment (start 100.325 64.685) (end 102.023 64.685) (width 0.254) (layer "B.Cu") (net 12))
 (segment (start 103.632 64.77) (end 103.632 68.58) (width 0.254) (layer "B.Cu") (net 12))
 (segment (start 102.108 64.77) (end 103.632 64.77) (width 0.254) (layer "B.Cu") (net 12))
 (segment (start 87.192 69.892) (end 96.007 70.019) (width 0.254) (layer "F.Cu") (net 24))
 (segment (start 96.007 70.019) (end 96.007 63.034) (width 0.254) (layer "F.Cu") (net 24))
 (segment (start 96.007 63.034) (end 97.785 62.145) (width 0.254) (layer "F.Cu") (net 24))
 (segment (start 85.935 68.635) (end 87.192 69.892) (width 0.254) (layer "F.Cu") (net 24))
 (segment (start 88.238 68.622) (end 94.991 68.622) (width 0.254) (layer "F.Cu") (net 23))
 (segment (start 88.225 68.635) (end 88.238 68.622) (width 0.254) (layer "F.Cu") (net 23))
 (via (at 94.991 68.622) (size 0.889) (drill 0.635) (layers "F.Cu" "B.Cu") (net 23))
 (segment (start 102.023 62.145) (end 102.108 62.23) (width 0.254) (layer "B.Cu") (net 23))
 (segment (start 95.038 68.622) (end 96.774 70.358) (width 0.254) (layer "B.Cu") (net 23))
 (segment (start 96.774 70.358) (end 104.394 70.358) (width 0.254) (layer "B.Cu") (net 23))
 (segment (start 104.394 70.358) (end 104.394 62.992) (width 0.254) (layer "B.Cu") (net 23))
 (segment (start 104.394 62.992) (end 103.632 62.23) (width 0.254) (layer "B.Cu") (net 23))
 (segment (start 100.325 62.145) (end 102.023 62.145) (width 0.254) (layer "B.Cu") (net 23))
 (segment (start 94.991 68.622) (end 95.038 68.622) (width 0.254) (layer "B.Cu") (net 23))
 (segment (start 102.108 62.23) (end 103.632 62.23) (width 0.254) (layer "B.Cu") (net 23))
 (segment (start 64.516 74.205) (end 72.385 66.336) (width 0.254) (layer "F.Cu") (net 11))
 (segment (start 72.385 66.336) (end 72.385 64.685) (width 0.254) (layer "F.Cu") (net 11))
 (segment (start 63.241 74.659) (end 63.241 78.528) (width 0.254) (layer "F.Cu") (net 11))
 (segment (start 63.241 78.528) (end 64.511 79.798) (width 0.254) (layer "F.Cu") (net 11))
 (segment (start 64.511 79.798) (end 78.989 79.798) (width 0.254) (layer "F.Cu") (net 11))
 (segment (start 78.989 79.798) (end 80.259 78.528) (width 0.254) (layer "F.Cu") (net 11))
 (segment (start 80.259 78.528) (end 80.259 74.569) (width 0.254) (layer "F.Cu") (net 11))
 (segment (start 80.259 74.569) (end 79.895 74.205) (width 0.254) (layer "F.Cu") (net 11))
 (segment (start 63.695 74.205) (end 63.241 74.659) (width 0.254) (layer "F.Cu") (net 11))
 (segment (start 63.695 74.205) (end 64.516 74.205) (width 0.254) (layer "F.Cu") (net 11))
 (segment (start 84.323 74.577) (end 84.323 78.655) (width 0.254) (layer "F.Cu") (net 22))
 (segment (start 84.323 78.655) (end 85.593 79.925) (width 0.254) (layer "F.Cu") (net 22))
 (segment (start 85.593 79.925) (end 100.071 79.925) (width 0.254) (layer "F.Cu") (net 22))
 (segment (start 100.071 79.925) (end 101.341 78.655) (width 0.254) (layer "F.Cu") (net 22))
 (segment (start 101.341 78.655) (end 101.341 74.651) (width 0.254) (layer "F.Cu") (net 22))
 (segment (start 101.341 74.651) (end 100.895 74.205) (width 0.254) (layer "F.Cu") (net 22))
 (segment (start 84.695 74.205) (end 84.323 74.577) (width 0.254) (layer "F.Cu") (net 22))
 (segment (start 84.577 74.087) (end 84.695 74.205) (width 0.254) (layer "B.Cu") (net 22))
 (segment (start 84.732 72.1806) (end 79.751 67.1996) (width 0.254) (layer "B.Cu") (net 22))
 (segment (start 79.751 67.1996) (end 79.0906 67.1996) (width 0.254) (layer "B.Cu") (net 22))
 (segment (start 79.0906 67.1996) (end 78.5318 66.6408) (width 0.254) (layer "B.Cu") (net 22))
 (segment (start 78.5318 66.6408) (end 76.7538 66.6408) (width 0.254) (layer "B.Cu") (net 22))
 (segment (start 76.7538 66.6408) (end 76.2204 66.1074) (width 0.254) (layer "B.Cu") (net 22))
 (segment (start 76.2204 66.1074) (end 74.417 66.1074) (width 0.254) (layer "B.Cu") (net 22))
 (segment (start 74.417 66.1074) (end 73.655 65.3454) (width 0.254) (layer "B.Cu") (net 22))
 (segment (start 73.655 65.3454) (end 73.655 63.415) (width 0.254) (layer "B.Cu") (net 22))
 (segment (start 73.655 63.415) (end 72.385 62.145) (width 0.254) (layer "B.Cu") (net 22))
 (segment (start 84.732 74.209) (end 84.732 72.1806) (width 0.254) (layer "B.Cu") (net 22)))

